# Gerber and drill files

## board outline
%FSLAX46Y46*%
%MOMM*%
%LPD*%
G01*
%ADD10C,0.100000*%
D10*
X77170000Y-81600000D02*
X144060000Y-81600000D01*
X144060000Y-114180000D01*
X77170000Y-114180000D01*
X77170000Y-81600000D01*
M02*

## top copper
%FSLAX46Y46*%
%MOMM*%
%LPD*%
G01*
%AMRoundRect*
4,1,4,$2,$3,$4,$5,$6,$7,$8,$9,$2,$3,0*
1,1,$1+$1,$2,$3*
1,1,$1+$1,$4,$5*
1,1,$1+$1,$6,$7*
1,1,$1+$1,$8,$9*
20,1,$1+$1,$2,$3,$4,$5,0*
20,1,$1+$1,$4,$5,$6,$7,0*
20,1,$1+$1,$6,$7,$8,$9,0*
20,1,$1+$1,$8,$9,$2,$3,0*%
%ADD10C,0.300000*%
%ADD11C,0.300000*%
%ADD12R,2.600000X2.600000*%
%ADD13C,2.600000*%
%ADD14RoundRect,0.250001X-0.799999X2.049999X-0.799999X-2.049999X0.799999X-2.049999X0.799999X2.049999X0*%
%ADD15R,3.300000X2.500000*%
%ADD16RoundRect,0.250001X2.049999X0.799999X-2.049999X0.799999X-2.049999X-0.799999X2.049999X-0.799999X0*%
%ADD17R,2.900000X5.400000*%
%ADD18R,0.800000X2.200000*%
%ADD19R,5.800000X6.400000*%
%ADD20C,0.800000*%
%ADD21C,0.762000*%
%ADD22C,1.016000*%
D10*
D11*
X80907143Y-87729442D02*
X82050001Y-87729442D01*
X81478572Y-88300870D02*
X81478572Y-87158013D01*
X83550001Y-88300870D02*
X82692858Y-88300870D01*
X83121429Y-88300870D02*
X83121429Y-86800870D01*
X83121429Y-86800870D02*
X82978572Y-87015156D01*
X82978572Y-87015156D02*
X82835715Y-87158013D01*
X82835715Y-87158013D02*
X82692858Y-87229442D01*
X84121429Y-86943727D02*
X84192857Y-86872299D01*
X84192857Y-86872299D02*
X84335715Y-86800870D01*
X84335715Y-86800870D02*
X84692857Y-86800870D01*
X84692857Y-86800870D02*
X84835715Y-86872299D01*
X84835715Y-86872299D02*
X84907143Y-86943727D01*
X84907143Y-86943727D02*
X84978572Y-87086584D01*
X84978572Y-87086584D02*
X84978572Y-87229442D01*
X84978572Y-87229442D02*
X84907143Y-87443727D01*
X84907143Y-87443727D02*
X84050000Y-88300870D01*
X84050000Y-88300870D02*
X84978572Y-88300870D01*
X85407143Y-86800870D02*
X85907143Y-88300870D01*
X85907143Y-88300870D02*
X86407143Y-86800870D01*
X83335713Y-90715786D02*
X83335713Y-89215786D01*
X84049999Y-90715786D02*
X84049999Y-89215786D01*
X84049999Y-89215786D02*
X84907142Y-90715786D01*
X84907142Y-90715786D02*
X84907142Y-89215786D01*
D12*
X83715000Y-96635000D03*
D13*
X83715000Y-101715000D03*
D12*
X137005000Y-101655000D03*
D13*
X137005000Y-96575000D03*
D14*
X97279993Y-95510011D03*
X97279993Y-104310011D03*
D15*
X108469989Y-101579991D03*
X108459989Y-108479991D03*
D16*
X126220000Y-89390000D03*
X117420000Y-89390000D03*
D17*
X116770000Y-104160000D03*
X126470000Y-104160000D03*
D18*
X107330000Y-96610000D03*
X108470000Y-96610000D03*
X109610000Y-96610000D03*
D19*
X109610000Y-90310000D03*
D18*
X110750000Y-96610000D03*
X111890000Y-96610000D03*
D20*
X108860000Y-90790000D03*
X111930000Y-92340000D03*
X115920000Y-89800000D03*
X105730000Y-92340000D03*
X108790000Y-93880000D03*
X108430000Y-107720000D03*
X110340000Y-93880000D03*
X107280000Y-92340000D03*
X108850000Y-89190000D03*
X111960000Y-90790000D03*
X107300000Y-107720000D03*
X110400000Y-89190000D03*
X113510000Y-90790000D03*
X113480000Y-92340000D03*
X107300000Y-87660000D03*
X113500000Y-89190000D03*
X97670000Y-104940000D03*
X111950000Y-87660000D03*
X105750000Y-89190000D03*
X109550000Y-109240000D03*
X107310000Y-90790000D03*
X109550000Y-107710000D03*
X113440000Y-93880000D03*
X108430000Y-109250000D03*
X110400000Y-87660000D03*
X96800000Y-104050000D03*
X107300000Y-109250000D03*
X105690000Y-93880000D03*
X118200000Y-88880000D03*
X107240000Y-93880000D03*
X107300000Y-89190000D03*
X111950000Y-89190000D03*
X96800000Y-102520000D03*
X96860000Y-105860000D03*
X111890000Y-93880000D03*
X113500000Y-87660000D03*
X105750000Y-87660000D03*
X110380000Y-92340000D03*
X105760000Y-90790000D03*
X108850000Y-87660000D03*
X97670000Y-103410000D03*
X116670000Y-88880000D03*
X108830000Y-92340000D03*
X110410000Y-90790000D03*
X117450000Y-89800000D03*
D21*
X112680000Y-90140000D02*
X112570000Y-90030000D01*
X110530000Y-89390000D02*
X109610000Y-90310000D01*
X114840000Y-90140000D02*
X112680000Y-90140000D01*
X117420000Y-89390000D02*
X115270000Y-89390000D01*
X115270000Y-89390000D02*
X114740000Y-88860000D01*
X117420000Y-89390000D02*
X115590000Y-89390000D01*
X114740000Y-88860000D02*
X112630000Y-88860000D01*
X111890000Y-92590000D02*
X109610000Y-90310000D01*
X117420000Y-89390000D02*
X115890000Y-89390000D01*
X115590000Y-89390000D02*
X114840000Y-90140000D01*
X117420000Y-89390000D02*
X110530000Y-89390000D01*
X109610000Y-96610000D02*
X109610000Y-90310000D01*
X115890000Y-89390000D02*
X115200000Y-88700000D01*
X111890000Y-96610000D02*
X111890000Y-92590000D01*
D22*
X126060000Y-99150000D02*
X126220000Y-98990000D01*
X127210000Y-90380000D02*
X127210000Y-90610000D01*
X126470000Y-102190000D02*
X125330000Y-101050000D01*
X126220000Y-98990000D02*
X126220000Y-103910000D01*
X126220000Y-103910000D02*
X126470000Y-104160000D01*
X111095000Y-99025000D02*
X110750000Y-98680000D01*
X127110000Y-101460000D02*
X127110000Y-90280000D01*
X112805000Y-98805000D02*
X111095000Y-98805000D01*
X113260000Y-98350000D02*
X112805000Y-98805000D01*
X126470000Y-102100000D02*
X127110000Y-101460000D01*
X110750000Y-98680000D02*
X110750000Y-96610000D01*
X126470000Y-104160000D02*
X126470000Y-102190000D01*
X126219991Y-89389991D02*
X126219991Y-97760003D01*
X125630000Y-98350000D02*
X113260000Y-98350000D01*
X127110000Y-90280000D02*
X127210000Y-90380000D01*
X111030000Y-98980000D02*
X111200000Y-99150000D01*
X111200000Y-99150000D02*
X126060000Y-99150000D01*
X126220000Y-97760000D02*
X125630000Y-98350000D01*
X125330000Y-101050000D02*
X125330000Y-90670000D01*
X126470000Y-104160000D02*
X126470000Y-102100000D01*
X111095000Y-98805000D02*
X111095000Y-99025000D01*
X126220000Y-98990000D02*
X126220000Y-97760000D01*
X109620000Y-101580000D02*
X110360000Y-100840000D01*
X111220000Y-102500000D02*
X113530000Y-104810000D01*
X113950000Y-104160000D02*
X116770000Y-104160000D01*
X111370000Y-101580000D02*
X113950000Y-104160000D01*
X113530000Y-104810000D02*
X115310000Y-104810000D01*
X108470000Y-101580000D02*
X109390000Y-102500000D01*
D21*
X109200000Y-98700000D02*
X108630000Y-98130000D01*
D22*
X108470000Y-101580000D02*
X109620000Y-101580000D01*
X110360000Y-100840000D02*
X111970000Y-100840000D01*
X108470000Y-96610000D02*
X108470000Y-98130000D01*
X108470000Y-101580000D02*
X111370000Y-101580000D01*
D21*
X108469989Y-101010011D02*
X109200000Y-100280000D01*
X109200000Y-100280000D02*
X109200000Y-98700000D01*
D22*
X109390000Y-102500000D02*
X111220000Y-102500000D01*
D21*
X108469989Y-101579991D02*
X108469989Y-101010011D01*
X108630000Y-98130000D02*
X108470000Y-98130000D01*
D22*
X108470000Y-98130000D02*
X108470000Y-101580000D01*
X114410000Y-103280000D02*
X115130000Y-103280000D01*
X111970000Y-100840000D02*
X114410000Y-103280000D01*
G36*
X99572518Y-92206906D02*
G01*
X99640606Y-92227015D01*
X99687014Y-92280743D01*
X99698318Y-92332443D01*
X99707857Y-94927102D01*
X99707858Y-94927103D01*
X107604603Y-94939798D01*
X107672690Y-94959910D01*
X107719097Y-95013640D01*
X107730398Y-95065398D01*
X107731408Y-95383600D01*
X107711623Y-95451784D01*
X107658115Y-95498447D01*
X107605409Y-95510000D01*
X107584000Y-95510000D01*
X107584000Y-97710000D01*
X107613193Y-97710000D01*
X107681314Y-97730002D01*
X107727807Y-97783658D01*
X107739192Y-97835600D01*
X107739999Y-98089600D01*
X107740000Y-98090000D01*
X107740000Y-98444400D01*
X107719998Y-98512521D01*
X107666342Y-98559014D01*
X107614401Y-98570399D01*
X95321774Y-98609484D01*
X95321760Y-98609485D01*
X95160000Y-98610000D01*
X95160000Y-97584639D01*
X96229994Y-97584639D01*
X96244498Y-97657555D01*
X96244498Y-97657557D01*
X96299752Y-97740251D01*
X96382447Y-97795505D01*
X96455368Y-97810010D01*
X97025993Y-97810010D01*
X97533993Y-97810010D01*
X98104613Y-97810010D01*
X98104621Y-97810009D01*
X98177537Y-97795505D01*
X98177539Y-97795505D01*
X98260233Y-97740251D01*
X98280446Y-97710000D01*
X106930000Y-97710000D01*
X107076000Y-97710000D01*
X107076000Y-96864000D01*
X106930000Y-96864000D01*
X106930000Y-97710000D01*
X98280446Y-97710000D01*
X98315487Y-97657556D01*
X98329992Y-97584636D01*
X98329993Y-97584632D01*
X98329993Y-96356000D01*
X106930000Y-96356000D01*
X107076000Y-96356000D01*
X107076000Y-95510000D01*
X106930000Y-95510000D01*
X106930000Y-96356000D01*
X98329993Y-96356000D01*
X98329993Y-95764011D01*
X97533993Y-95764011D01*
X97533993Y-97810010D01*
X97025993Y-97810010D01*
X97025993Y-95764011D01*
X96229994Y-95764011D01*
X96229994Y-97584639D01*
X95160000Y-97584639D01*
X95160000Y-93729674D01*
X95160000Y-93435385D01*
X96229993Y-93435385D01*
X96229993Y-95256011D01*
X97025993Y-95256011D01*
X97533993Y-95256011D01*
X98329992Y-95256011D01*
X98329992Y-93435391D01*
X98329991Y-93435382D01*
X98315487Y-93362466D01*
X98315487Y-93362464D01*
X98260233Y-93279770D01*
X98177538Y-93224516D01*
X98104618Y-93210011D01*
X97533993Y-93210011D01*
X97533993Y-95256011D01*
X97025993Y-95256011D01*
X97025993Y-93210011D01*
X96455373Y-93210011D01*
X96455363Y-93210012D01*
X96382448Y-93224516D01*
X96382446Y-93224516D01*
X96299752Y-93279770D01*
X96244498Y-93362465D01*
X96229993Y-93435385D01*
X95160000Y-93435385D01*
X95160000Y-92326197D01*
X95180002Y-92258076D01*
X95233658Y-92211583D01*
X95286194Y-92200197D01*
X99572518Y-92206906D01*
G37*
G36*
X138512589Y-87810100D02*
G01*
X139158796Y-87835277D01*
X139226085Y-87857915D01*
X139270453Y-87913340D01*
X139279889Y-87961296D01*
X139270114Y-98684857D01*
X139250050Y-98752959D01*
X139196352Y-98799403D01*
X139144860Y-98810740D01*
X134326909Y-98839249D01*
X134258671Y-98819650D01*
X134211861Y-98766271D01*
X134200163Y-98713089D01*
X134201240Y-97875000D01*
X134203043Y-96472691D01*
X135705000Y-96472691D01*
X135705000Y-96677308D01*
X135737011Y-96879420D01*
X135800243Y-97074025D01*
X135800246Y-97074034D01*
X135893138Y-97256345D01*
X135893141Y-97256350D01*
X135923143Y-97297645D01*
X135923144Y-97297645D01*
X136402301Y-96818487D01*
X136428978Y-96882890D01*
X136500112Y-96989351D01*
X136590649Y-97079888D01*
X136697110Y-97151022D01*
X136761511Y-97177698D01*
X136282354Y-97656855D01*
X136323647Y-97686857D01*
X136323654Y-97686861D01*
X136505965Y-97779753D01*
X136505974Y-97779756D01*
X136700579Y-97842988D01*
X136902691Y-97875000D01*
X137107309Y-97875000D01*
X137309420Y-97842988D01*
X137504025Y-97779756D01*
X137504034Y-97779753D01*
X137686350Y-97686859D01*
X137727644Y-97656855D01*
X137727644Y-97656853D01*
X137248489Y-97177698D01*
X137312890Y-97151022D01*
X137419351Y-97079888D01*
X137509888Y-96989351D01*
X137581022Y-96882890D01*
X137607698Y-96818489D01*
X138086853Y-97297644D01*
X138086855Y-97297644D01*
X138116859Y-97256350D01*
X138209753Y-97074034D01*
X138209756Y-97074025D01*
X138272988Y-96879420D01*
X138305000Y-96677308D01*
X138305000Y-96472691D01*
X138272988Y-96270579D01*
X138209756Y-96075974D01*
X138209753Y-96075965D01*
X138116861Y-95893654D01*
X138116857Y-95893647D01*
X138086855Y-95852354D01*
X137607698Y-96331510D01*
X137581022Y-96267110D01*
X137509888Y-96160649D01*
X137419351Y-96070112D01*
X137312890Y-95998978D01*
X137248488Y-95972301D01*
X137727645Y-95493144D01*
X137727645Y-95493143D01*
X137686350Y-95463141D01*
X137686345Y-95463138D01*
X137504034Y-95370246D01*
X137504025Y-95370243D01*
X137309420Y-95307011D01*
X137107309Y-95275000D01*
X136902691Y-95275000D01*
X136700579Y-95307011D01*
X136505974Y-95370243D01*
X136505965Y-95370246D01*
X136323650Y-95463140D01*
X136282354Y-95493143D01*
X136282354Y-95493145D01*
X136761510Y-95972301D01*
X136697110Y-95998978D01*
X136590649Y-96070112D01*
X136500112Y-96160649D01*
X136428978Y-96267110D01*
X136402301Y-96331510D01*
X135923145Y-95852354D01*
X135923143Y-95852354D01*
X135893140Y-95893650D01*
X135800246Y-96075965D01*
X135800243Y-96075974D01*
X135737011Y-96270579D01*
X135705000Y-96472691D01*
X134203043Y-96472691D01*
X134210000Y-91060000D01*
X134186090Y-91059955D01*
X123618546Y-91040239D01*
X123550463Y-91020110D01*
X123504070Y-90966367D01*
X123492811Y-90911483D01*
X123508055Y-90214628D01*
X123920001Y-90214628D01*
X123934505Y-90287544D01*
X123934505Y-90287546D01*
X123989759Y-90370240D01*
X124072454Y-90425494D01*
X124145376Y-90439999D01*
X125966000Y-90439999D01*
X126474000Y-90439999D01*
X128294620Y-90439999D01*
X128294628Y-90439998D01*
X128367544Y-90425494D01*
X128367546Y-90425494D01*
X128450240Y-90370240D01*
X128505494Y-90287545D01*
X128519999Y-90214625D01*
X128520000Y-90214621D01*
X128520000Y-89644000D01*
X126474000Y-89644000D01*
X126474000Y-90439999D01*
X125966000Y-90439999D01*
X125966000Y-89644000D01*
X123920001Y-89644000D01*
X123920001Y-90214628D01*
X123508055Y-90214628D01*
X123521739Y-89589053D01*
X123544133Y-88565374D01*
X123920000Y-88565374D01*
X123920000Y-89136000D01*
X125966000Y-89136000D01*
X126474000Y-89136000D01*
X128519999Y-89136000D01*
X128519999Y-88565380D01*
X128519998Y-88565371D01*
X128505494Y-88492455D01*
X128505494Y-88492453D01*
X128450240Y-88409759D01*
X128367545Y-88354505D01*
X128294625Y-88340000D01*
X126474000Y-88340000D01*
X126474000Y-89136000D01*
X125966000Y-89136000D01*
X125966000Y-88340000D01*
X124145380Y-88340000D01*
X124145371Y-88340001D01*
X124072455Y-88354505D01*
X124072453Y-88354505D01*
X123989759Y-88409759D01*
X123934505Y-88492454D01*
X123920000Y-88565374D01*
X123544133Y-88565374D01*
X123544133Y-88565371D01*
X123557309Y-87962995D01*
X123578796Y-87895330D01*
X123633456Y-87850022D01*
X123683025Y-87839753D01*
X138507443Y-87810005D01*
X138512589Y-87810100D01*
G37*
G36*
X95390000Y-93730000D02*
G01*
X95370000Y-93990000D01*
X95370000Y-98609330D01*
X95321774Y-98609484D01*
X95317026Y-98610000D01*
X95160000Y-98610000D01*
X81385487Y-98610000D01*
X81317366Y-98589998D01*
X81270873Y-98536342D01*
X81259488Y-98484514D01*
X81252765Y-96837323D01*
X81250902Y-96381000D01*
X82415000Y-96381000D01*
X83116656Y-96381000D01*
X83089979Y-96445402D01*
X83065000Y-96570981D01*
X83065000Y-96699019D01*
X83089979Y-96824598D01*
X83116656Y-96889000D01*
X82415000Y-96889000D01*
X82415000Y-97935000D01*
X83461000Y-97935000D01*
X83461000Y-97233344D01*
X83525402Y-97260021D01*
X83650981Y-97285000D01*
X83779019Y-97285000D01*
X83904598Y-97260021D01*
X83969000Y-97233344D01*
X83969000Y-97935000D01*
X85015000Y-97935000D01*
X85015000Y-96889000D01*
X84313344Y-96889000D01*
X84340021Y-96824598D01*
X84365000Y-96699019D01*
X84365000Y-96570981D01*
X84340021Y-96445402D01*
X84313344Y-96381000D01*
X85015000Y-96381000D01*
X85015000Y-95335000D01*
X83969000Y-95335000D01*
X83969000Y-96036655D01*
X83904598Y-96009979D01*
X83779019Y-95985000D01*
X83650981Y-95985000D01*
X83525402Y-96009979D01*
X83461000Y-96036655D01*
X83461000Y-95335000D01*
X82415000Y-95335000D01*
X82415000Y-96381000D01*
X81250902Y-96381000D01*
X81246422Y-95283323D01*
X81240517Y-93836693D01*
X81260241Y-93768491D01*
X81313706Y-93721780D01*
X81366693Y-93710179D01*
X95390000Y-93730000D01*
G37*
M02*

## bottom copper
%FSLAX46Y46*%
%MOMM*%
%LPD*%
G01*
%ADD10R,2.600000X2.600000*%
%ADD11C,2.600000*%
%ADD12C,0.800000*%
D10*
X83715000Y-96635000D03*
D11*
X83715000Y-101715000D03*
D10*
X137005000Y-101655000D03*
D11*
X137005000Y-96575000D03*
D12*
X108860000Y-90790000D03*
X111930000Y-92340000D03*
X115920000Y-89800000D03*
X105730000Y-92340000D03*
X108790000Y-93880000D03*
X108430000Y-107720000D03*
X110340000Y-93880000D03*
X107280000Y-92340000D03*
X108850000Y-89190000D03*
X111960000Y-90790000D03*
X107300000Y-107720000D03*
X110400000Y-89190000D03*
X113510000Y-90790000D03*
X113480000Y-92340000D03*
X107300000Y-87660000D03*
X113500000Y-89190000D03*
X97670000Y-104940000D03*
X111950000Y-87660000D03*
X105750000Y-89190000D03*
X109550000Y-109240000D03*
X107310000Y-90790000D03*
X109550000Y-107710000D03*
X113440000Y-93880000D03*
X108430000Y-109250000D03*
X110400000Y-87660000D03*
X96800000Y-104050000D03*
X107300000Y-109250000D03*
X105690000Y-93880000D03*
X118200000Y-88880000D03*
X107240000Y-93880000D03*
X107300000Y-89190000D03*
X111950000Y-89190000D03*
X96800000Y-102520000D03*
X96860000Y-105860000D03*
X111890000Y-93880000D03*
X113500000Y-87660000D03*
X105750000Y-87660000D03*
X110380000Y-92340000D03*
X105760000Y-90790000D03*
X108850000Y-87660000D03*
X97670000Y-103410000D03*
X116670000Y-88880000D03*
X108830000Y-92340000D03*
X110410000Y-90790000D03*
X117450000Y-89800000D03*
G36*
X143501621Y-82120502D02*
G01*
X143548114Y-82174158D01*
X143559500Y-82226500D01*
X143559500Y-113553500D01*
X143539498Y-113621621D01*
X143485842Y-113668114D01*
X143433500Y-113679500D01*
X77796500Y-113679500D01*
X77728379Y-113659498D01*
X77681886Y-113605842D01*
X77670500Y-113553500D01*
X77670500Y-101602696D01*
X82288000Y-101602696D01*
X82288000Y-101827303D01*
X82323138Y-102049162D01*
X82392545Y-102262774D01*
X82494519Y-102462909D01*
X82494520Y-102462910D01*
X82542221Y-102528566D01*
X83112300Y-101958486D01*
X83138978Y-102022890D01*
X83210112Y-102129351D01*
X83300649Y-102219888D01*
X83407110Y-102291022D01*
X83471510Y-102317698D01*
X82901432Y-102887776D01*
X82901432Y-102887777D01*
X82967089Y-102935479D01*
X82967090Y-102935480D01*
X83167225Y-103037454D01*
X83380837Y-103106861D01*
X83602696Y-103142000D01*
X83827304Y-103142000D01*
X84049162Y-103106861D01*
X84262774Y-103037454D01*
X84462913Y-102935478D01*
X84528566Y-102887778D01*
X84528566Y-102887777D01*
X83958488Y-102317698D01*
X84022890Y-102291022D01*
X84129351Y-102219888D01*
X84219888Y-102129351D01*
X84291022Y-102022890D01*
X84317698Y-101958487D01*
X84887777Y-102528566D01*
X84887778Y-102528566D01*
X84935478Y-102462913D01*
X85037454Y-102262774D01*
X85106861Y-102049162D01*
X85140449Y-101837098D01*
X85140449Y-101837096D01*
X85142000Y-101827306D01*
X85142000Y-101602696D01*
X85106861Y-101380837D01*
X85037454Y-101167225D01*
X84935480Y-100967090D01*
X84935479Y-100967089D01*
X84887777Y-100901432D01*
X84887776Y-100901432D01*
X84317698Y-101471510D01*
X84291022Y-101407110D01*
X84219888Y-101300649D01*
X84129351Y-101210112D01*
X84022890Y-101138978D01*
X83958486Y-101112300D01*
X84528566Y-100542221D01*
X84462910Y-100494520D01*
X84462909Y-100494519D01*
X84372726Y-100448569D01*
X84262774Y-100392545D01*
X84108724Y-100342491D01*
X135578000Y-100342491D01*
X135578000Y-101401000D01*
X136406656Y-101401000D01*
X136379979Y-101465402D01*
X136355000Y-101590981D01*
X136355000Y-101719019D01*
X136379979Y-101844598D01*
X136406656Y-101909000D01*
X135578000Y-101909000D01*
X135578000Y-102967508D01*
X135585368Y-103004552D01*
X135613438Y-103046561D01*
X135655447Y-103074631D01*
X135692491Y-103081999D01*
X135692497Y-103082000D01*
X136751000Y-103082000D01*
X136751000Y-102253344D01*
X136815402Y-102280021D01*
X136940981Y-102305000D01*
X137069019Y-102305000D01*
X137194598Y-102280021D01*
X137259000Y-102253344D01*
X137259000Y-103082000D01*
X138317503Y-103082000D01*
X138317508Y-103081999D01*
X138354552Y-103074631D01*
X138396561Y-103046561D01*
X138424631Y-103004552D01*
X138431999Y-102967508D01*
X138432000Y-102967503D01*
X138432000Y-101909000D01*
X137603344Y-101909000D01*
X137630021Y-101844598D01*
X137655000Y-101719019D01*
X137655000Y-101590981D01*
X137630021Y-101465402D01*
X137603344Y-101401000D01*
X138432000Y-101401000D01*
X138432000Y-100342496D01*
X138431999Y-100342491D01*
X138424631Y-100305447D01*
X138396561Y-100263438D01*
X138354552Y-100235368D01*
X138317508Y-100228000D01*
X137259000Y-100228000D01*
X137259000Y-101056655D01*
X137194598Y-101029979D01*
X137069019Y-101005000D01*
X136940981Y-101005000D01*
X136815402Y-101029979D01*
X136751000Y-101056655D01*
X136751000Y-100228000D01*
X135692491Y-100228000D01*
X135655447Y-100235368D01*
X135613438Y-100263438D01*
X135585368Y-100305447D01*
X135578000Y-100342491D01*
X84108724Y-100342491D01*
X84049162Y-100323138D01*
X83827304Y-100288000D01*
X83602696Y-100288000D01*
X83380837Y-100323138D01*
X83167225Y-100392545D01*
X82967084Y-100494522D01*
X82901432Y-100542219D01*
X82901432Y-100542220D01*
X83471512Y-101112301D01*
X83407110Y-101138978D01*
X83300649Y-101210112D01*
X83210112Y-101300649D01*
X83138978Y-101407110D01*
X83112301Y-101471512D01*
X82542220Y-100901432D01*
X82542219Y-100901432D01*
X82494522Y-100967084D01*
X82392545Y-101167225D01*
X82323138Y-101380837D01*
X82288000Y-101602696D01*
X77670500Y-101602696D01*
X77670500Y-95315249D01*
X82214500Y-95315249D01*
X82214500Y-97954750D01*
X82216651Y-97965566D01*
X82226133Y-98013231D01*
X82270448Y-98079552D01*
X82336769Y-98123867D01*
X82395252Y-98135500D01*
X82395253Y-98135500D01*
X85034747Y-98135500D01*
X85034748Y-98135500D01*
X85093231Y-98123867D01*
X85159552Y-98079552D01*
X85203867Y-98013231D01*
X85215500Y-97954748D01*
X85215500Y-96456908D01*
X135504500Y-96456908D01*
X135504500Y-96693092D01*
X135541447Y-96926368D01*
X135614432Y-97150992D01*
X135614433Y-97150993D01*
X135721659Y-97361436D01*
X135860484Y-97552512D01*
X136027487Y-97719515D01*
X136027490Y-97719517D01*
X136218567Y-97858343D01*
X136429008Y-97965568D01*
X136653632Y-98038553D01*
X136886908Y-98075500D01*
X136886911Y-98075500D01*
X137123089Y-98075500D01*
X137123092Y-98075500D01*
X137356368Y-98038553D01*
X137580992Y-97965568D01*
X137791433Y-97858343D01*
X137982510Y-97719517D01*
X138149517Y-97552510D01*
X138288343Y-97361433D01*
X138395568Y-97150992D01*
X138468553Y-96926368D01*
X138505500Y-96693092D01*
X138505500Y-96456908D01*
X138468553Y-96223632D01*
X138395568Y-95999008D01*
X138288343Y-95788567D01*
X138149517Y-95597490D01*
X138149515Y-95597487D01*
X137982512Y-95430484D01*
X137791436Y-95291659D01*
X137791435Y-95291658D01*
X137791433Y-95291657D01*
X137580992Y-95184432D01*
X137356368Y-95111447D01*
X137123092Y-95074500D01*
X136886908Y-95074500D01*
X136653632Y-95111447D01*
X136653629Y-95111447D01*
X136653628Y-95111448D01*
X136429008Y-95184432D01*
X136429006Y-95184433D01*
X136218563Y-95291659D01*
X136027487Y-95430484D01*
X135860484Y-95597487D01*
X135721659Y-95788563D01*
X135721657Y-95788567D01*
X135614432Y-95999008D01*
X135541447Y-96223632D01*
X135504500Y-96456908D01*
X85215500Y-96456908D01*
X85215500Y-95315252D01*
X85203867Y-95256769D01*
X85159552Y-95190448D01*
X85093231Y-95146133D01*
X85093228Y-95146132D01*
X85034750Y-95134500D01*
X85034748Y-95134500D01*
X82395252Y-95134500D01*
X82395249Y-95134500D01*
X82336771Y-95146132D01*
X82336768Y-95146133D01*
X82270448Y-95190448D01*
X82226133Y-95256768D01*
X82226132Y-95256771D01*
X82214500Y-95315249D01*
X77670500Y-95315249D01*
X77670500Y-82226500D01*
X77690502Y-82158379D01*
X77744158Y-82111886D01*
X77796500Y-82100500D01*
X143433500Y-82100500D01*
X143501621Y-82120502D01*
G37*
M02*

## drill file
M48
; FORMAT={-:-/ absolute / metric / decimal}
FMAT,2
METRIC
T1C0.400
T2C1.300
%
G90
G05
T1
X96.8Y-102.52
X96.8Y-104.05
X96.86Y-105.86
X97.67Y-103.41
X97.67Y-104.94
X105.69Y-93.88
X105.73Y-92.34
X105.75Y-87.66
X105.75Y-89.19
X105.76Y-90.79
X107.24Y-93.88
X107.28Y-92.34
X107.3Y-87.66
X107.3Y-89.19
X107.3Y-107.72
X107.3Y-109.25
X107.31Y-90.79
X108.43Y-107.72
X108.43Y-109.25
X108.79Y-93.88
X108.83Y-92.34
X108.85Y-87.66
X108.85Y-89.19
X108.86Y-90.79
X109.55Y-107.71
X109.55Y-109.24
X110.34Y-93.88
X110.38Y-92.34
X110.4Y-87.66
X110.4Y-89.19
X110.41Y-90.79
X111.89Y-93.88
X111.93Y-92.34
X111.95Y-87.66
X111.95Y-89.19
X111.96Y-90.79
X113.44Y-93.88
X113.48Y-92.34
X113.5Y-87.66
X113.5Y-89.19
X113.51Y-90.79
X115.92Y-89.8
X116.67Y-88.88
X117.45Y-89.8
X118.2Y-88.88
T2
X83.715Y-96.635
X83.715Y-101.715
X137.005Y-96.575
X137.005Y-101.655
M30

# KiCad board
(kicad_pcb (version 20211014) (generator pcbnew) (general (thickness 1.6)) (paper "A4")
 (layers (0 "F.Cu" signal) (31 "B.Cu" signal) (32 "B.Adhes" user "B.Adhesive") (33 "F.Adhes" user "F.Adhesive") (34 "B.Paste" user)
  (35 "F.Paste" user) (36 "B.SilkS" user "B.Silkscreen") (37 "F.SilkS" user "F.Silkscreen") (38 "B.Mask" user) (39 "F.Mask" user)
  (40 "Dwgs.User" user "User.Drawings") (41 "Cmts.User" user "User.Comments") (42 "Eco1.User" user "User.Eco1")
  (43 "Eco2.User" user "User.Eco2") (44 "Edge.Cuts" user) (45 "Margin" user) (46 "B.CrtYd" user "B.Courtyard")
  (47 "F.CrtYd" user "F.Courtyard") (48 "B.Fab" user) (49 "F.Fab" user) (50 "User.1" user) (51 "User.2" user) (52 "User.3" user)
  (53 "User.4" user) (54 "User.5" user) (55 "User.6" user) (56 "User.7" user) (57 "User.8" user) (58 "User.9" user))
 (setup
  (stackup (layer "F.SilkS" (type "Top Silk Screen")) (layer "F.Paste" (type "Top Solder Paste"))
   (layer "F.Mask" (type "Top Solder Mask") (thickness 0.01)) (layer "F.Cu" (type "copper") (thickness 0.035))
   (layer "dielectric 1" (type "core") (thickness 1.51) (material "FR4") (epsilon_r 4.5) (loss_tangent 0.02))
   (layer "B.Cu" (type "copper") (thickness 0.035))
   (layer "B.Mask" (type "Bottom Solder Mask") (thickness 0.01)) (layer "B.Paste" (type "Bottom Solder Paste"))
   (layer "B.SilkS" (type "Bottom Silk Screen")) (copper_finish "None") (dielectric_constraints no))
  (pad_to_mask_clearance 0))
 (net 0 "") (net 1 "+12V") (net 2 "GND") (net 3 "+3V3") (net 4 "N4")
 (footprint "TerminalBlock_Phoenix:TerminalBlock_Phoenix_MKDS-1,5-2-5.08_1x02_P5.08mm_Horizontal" (layer "F.Cu") (at 83.715 96.635 -90)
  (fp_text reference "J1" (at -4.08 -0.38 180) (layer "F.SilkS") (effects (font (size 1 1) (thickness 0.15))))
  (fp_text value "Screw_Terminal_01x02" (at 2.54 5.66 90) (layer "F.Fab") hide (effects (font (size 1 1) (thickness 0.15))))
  (pad "1" thru_hole rect locked (at 0 0 270) (size 2.6 2.6) (drill 1.3) (layers *.Cu *.Mask) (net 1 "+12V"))
  (pad "2" thru_hole circle locked (at 5.08 0 270) (size 2.6 2.6) (drill 1.3) (layers *.Cu *.Mask) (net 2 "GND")))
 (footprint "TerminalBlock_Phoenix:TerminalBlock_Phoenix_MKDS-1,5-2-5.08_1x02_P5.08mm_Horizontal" (layer "F.Cu") (at 137.005 101.655 90)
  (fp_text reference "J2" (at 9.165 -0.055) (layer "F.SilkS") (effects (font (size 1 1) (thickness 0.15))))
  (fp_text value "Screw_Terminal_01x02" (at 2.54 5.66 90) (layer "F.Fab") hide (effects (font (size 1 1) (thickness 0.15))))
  (pad "1" thru_hole rect locked (at 0 0 90) (size 2.6 2.6) (drill 1.3) (layers *.Cu *.Mask) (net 2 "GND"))
  (pad "2" thru_hole circle locked (at 5.08 0 90) (size 2.6 2.6) (drill 1.3) (layers *.Cu *.Mask) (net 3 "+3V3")))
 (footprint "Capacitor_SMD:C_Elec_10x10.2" (layer "F.Cu") (at 97.279993 99.910011 -90)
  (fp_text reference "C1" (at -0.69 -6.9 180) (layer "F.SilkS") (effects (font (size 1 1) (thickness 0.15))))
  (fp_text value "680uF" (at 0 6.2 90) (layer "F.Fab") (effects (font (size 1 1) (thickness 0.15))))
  (pad "1" smd roundrect locked (at -4.4 0 270) (size 4.6 2.1) (layers "F.Cu" "F.Paste" "F.Mask") (roundrect_rratio 0.119048) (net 1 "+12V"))
  (pad "2" smd roundrect locked (at 4.4 0 270) (size 4.6 2.1) (layers "F.Cu" "F.Paste" "F.Mask") (roundrect_rratio 0.119048) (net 2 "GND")))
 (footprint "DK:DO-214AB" (layer "F.Cu") (at 108.469989 105.029991 -90)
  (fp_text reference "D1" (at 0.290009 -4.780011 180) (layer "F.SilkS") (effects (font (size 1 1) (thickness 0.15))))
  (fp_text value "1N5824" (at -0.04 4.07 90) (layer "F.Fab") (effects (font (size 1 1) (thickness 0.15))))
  (pad "1" smd rect locked (at -3.45 0 270) (size 2.5 3.3) (layers "F.Cu" "F.Paste" "F.Mask") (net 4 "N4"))
  (pad "2" smd rect locked (at 3.45 0.01 270) (size 2.5 3.3) (layers "F.Cu" "F.Paste" "F.Mask") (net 2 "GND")))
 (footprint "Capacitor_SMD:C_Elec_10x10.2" (layer "F.Cu") (at 121.82 89.39 180)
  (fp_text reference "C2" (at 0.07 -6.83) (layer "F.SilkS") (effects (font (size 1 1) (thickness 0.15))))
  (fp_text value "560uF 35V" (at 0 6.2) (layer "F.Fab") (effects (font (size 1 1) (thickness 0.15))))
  (pad "1" smd roundrect locked (at -4.4 0 180) (size 4.6 2.1) (layers "F.Cu" "F.Paste" "F.Mask") (roundrect_rratio 0.119048) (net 3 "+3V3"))
  (pad "2" smd roundrect locked (at 4.4 0 180) (size 4.6 2.1) (layers "F.Cu" "F.Paste" "F.Mask") (roundrect_rratio 0.119048) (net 2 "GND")))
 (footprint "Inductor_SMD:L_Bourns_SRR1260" (layer "F.Cu") (at 121.62 104.16)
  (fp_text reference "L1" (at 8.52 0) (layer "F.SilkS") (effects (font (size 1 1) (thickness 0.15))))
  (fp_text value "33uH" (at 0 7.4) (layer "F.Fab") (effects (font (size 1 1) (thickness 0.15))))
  (pad "1" smd rect locked (at -4.85 0) (size 2.9 5.4) (layers "F.Cu" "F.Paste" "F.Mask") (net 4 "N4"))
  (pad "2" smd rect locked (at 4.85 0) (size 2.9 5.4) (layers "F.Cu" "F.Paste" "F.Mask") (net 3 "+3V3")))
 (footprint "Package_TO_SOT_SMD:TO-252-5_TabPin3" (layer "F.Cu") (at 109.61 92.41 90)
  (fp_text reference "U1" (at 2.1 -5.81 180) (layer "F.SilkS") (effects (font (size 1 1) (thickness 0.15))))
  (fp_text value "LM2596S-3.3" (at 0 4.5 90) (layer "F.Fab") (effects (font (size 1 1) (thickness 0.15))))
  (pad "" smd rect locked (at 3.775 1.525 90) (size 3.05 2.75) (layers "F.Paste"))
  (pad "" smd rect locked (at 0.425 -1.525 90) (size 3.05 2.75) (layers "F.Paste"))
  (pad "" smd rect locked (at 0.425 1.525 90) (size 3.05 2.75) (layers "F.Paste"))
  (pad "" smd rect locked (at 3.775 -1.525 90) (size 3.05 2.75) (layers "F.Paste"))
  (pad "1" smd rect locked (at -4.2 -2.28 90) (size 2.2 0.8) (layers "F.Cu" "F.Paste" "F.Mask") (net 1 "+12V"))
  (pad "2" smd rect locked (at -4.2 -1.14 90) (size 2.2 0.8) (layers "F.Cu" "F.Paste" "F.Mask") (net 4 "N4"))
  (pad "3" smd rect locked (at -4.2 0 90) (size 2.2 0.8) (layers "F.Cu" "F.Paste" "F.Mask") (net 2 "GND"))
  (pad "3" smd rect locked (at 2.1 0 90) (size 6.4 5.8) (layers "F.Cu" "F.Mask") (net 2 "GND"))
  (pad "4" smd rect locked (at -4.2 1.14 90) (size 2.2 0.8) (layers "F.Cu" "F.Paste" "F.Mask") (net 3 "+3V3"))
  (pad "5" smd rect locked (at -4.2 2.28 90) (size 2.2 0.8) (layers "F.Cu" "F.Paste" "F.Mask") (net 2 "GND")))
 (gr_rect (start 77.17 81.6) (end 144.06 114.18) (layer "Edge.Cuts") (width 0.1) (fill none))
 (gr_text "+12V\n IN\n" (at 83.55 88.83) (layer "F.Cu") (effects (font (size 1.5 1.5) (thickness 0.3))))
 (segment (start 112.68 90.14) (end 112.57 90.03) (width 0.762) (layer "F.Cu") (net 2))
 (segment (start 110.53 89.39) (end 109.61 90.31) (width 0.762) (layer "F.Cu") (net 2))
 (segment (start 114.84 90.14) (end 112.68 90.14) (width 0.762) (layer "F.Cu") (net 2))
 (segment (start 117.42 89.39) (end 115.27 89.39) (width 0.762) (layer "F.Cu") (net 2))
 (segment (start 115.27 89.39) (end 114.74 88.86) (width 0.762) (layer "F.Cu") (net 2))
 (segment (start 117.42 89.39) (end 115.59 89.39) (width 0.762) (layer "F.Cu") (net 2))
 (segment (start 114.74 88.86) (end 112.63 88.86) (width 0.762) (layer "F.Cu") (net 2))
 (segment (start 111.89 92.59) (end 109.61 90.31) (width 0.762) (layer "F.Cu") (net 2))
 (segment (start 117.42 89.39) (end 115.89 89.39) (width 0.762) (layer "F.Cu") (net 2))
 (segment (start 115.59 89.39) (end 114.84 90.14) (width 0.762) (layer "F.Cu") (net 2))
 (segment (start 117.42 89.39) (end 110.53 89.39) (width 0.762) (layer "F.Cu") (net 2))
 (segment (start 109.61 96.61) (end 109.61 90.31) (width 0.762) (layer "F.Cu") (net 2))
 (segment (start 115.89 89.39) (end 115.2 88.7) (width 0.762) (layer "F.Cu") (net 2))
 (segment (start 111.89 96.61) (end 111.89 92.59) (width 0.762) (layer "F.Cu") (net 2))
 (via (at 108.86 90.79) (size 0.8) (drill 0.4) (layers "F.Cu" "B.Cu") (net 2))
 (via (at 111.93 92.34) (size 0.8) (drill 0.4) (layers "F.Cu" "B.Cu") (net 2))
 (via (at 115.92 89.8) (size 0.8) (drill 0.4) (layers "F.Cu" "B.Cu") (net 2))
 (via (at 105.73 92.34) (size 0.8) (drill 0.4) (layers "F.Cu" "B.Cu") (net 2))
 (via (at 108.79 93.88) (size 0.8) (drill 0.4) (layers "F.Cu" "B.Cu") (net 2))
 (via (at 108.43 107.72) (size 0.8) (drill 0.4) (layers "F.Cu" "B.Cu") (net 2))
 (via (at 110.34 93.88) (size 0.8) (drill 0.4) (layers "F.Cu" "B.Cu") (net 2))
 (via (at 107.28 92.34) (size 0.8) (drill 0.4) (layers "F.Cu" "B.Cu") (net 2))
 (via (at 108.85 89.19) (size 0.8) (drill 0.4) (layers "F.Cu" "B.Cu") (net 2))
 (via (at 111.96 90.79) (size 0.8) (drill 0.4) (layers "F.Cu" "B.Cu") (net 2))
 (via (at 107.3 107.72) (size 0.8) (drill 0.4) (layers "F.Cu" "B.Cu") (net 2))
 (via (at 110.4 89.19) (size 0.8) (drill 0.4) (layers "F.Cu" "B.Cu") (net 2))
 (via (at 113.51 90.79) (size 0.8) (drill 0.4) (layers "F.Cu" "B.Cu") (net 2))
 (via (at 113.48 92.34) (size 0.8) (drill 0.4) (layers "F.Cu" "B.Cu") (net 2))
 (via (at 107.3 87.66) (size 0.8) (drill 0.4) (layers "F.Cu" "B.Cu") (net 2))
 (via (at 113.5 89.19) (size 0.8) (drill 0.4) (layers "F.Cu" "B.Cu") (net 2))
 (via (at 97.67 104.94) (size 0.8) (drill 0.4) (layers "F.Cu" "B.Cu") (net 2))
 (via (at 111.95 87.66) (size 0.8) (drill 0.4) (layers "F.Cu" "B.Cu") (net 2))
 (via (at 105.75 89.19) (size 0.8) (drill 0.4) (layers "F.Cu" "B.Cu") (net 2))
 (via (at 109.55 109.24) (size 0.8) (drill 0.4) (layers "F.Cu" "B.Cu") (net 2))
 (via (at 107.31 90.79) (size 0.8) (drill 0.4) (layers "F.Cu" "B.Cu") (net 2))
 (via (at 109.55 107.71) (size 0.8) (drill 0.4) (layers "F.Cu" "B.Cu") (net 2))
 (via (at 113.44 93.88) (size 0.8) (drill 0.4) (layers "F.Cu" "B.Cu") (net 2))
 (via (at 108.43 109.25) (size 0.8) (drill 0.4) (layers "F.Cu" "B.Cu") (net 2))
 (via (at 110.4 87.66) (size 0.8) (drill 0.4) (layers "F.Cu" "B.Cu") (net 2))
 (via (at 96.8 104.05) (size 0.8) (drill 0.4) (layers "F.Cu" "B.Cu") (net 2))
 (via (at 107.3 109.25) (size 0.8) (drill 0.4) (layers "F.Cu" "B.Cu") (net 2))
 (via (at 105.69 93.88) (size 0.8) (drill 0.4) (layers "F.Cu" "B.Cu") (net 2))
 (via (at 118.2 88.88) (size 0.8) (drill 0.4) (layers "F.Cu" "B.Cu") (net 2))
 (via (at 107.24 93.88) (size 0.8) (drill 0.4) (layers "F.Cu" "B.Cu") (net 2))
 (via (at 107.3 89.19) (size 0.8) (drill 0.4) (layers "F.Cu" "B.Cu") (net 2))
 (via (at 111.95 89.19) (size 0.8) (drill 0.4) (layers "F.Cu" "B.Cu") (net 2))
 (via (at 96.8 102.52) (size 0.8) (drill 0.4) (layers "F.Cu" "B.Cu") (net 2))
 (via (at 96.86 105.86) (size 0.8) (drill 0.4) (layers "F.Cu" "B.Cu") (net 2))
 (via (at 111.89 93.88) (size 0.8) (drill 0.4) (layers "F.Cu" "B.Cu") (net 2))
 (via (at 113.5 87.66) (size 0.8) (drill 0.4) (layers "F.Cu" "B.Cu") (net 2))
 (via (at 105.75 87.66) (size 0.8) (drill 0.4) (layers "F.Cu" "B.Cu") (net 2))
 (via (at 110.38 92.34) (size 0.8) (drill 0.4) (layers "F.Cu" "B.Cu") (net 2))
 (via (at 105.76 90.79) (size 0.8) (drill 0.4) (layers "F.Cu" "B.Cu") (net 2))
 (via (at 108.85 87.66) (size 0.8) (drill 0.4) (layers "F.Cu" "B.Cu") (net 2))
 (via (at 97.67 103.41) (size 0.8) (drill 0.4) (layers "F.Cu" "B.Cu") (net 2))
 (via (at 116.67 88.88) (size 0.8) (drill 0.4) (layers "F.Cu" "B.Cu") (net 2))
 (via (at 108.83 92.34) (size 0.8) (drill 0.4) (layers "F.Cu" "B.Cu") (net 2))
 (via (at 110.41 90.79) (size 0.8) (drill 0.4) (layers "F.Cu" "B.Cu") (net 2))
 (via (at 117.45 89.8) (size 0.8) (drill 0.4) (layers "F.Cu" "B.Cu") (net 2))
 (segment (start 126.06 99.15) (end 126.22 98.99) (width 1.016) (layer "F.Cu") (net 3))
 (segment (start 127.21 90.38) (end 127.21 90.61) (width 1.016) (layer "F.Cu") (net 3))
 (segment (start 126.47 102.19) (end 125.33 101.05) (width 1.016) (layer "F.Cu") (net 3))
 (segment (start 126.22 98.99) (end 126.22 103.91) (width 1.016) (layer "F.Cu") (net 3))
 (segment (start 126.22 103.91) (end 126.47 104.16) (width 1.016) (layer "F.Cu") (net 3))
 (segment (start 111.095 99.025) (end 110.75 98.68) (width 1.016) (layer "F.Cu") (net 3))
 (segment (start 127.11 101.46) (end 127.11 90.28) (width 1.016) (layer "F.Cu") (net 3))
 (segment (start 112.805 98.805) (end 111.095 98.805) (width 1.016) (layer "F.Cu") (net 3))
 (segment (start 113.26 98.35) (end 112.805 98.805) (width 1.016) (layer "F.Cu") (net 3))
 (segment (start 126.47 102.1) (end 127.11 101.46) (width 1.016) (layer "F.Cu") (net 3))
 (segment (start 110.75 98.68) (end 110.75 96.61) (width 1.016) (layer "F.Cu") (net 3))
 (segment (start 126.47 104.16) (end 126.47 102.19) (width 1.016) (layer "F.Cu") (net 3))
 (segment (start 126.219991 89.389991) (end 126.219991 97.760003) (width 1.016) (layer "F.Cu") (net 3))
 (segment (start 125.63 98.35) (end 113.26 98.35) (width 1.016) (layer "F.Cu") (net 3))
 (segment (start 127.11 90.28) (end 127.21 90.38) (width 1.016) (layer "F.Cu") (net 3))
 (segment (start 111.03 98.98) (end 111.2 99.15) (width 1.016) (layer "F.Cu") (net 3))
 (segment (start 111.2 99.15) (end 126.06 99.15) (width 1.016) (layer "F.Cu") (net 3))
 (segment (start 126.22 97.76) (end 125.63 98.35) (width 1.016) (layer "F.Cu") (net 3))
 (segment (start 125.33 101.05) (end 125.33 90.67) (width 1.016) (layer "F.Cu") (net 3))
 (segment (start 126.47 104.16) (end 126.47 102.1) (width 1.016) (layer "F.Cu") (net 3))
 (segment (start 111.095 98.805) (end 111.095 99.025) (width 1.016) (layer "F.Cu") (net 3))
 (segment (start 126.22 98.99) (end 126.22 97.76) (width 1.016) (layer "F.Cu") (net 3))
 (segment (start 109.62 101.58) (end 110.36 100.84) (width 1.016) (layer "F.Cu") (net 4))
 (segment (start 111.22 102.5) (end 113.53 104.81) (width 1.016) (layer "F.Cu") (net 4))
 (segment (start 113.95 104.16) (end 116.77 104.16) (width 1.016) (layer "F.Cu") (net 4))
 (segment (start 111.37 101.58) (end 113.95 104.16) (width 1.016) (layer "F.Cu") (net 4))
 (segment (start 113.53 104.81) (end 115.31 104.81) (width 1.016) (layer "F.Cu") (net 4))
 (segment (start 108.47 101.58) (end 109.39 102.5) (width 1.016) (layer "F.Cu") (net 4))
 (segment (start 109.2 98.7) (end 108.63 98.13) (width 0.762) (layer "F.Cu") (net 4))
 (segment (start 108.47 101.58) (end 109.62 101.58) (width 1.016) (layer "F.Cu") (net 4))
 (segment (start 110.36 100.84) (end 111.97 100.84) (width 1.016) (layer "F.Cu") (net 4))
 (segment (start 108.47 96.61) (end 108.47 98.13) (width 1.016) (layer "F.Cu") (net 4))
 (segment (start 108.47 101.58) (end 111.37 101.58) (width 1.016) (layer "F.Cu") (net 4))
 (segment (start 108.469989 101.010011) (end 109.2 100.28) (width 0.762) (layer "F.Cu") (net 4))
 (segment (start 109.2 100.28) (end 109.2 98.7) (width 0.762) (layer "F.Cu") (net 4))
 (segment (start 109.39 102.5) (end 111.22 102.5) (width 1.016) (layer "F.Cu") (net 4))
 (segment (start 108.469989 101.579991) (end 108.469989 101.010011) (width 0.762) (layer "F.Cu") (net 4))
 (segment (start 108.63 98.13) (end 108.47 98.13) (width 0.762) (layer "F.Cu") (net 4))
 (segment (start 108.47 98.13) (end 108.47 101.58) (width 1.016) (layer "F.Cu") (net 4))
 (segment (start 114.41 103.28) (end 115.13 103.28) (width 1.016) (layer "F.Cu") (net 4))
 (segment (start 111.97 100.84) (end 114.41 103.28) (width 1.016) (layer "F.Cu") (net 4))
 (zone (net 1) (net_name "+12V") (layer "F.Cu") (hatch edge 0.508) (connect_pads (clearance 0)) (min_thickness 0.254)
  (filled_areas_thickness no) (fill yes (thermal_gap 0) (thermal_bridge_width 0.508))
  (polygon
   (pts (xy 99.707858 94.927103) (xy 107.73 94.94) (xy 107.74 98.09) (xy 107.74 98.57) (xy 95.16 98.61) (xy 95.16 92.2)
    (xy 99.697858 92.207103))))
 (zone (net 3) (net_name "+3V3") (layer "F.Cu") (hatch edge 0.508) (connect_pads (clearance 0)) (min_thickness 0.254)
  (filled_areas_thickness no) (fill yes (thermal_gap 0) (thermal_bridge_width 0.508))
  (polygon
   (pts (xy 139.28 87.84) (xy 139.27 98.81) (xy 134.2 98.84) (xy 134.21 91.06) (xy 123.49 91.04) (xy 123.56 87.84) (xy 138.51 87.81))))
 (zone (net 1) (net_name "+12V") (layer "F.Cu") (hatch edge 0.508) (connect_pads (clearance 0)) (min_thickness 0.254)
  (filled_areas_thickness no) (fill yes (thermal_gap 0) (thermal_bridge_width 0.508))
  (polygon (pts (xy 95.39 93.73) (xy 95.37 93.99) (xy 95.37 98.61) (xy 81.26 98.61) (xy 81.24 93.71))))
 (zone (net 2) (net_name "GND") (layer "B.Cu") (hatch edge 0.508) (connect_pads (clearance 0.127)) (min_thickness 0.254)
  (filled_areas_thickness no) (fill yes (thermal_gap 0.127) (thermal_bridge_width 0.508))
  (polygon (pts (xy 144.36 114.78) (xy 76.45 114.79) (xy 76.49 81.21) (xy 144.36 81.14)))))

